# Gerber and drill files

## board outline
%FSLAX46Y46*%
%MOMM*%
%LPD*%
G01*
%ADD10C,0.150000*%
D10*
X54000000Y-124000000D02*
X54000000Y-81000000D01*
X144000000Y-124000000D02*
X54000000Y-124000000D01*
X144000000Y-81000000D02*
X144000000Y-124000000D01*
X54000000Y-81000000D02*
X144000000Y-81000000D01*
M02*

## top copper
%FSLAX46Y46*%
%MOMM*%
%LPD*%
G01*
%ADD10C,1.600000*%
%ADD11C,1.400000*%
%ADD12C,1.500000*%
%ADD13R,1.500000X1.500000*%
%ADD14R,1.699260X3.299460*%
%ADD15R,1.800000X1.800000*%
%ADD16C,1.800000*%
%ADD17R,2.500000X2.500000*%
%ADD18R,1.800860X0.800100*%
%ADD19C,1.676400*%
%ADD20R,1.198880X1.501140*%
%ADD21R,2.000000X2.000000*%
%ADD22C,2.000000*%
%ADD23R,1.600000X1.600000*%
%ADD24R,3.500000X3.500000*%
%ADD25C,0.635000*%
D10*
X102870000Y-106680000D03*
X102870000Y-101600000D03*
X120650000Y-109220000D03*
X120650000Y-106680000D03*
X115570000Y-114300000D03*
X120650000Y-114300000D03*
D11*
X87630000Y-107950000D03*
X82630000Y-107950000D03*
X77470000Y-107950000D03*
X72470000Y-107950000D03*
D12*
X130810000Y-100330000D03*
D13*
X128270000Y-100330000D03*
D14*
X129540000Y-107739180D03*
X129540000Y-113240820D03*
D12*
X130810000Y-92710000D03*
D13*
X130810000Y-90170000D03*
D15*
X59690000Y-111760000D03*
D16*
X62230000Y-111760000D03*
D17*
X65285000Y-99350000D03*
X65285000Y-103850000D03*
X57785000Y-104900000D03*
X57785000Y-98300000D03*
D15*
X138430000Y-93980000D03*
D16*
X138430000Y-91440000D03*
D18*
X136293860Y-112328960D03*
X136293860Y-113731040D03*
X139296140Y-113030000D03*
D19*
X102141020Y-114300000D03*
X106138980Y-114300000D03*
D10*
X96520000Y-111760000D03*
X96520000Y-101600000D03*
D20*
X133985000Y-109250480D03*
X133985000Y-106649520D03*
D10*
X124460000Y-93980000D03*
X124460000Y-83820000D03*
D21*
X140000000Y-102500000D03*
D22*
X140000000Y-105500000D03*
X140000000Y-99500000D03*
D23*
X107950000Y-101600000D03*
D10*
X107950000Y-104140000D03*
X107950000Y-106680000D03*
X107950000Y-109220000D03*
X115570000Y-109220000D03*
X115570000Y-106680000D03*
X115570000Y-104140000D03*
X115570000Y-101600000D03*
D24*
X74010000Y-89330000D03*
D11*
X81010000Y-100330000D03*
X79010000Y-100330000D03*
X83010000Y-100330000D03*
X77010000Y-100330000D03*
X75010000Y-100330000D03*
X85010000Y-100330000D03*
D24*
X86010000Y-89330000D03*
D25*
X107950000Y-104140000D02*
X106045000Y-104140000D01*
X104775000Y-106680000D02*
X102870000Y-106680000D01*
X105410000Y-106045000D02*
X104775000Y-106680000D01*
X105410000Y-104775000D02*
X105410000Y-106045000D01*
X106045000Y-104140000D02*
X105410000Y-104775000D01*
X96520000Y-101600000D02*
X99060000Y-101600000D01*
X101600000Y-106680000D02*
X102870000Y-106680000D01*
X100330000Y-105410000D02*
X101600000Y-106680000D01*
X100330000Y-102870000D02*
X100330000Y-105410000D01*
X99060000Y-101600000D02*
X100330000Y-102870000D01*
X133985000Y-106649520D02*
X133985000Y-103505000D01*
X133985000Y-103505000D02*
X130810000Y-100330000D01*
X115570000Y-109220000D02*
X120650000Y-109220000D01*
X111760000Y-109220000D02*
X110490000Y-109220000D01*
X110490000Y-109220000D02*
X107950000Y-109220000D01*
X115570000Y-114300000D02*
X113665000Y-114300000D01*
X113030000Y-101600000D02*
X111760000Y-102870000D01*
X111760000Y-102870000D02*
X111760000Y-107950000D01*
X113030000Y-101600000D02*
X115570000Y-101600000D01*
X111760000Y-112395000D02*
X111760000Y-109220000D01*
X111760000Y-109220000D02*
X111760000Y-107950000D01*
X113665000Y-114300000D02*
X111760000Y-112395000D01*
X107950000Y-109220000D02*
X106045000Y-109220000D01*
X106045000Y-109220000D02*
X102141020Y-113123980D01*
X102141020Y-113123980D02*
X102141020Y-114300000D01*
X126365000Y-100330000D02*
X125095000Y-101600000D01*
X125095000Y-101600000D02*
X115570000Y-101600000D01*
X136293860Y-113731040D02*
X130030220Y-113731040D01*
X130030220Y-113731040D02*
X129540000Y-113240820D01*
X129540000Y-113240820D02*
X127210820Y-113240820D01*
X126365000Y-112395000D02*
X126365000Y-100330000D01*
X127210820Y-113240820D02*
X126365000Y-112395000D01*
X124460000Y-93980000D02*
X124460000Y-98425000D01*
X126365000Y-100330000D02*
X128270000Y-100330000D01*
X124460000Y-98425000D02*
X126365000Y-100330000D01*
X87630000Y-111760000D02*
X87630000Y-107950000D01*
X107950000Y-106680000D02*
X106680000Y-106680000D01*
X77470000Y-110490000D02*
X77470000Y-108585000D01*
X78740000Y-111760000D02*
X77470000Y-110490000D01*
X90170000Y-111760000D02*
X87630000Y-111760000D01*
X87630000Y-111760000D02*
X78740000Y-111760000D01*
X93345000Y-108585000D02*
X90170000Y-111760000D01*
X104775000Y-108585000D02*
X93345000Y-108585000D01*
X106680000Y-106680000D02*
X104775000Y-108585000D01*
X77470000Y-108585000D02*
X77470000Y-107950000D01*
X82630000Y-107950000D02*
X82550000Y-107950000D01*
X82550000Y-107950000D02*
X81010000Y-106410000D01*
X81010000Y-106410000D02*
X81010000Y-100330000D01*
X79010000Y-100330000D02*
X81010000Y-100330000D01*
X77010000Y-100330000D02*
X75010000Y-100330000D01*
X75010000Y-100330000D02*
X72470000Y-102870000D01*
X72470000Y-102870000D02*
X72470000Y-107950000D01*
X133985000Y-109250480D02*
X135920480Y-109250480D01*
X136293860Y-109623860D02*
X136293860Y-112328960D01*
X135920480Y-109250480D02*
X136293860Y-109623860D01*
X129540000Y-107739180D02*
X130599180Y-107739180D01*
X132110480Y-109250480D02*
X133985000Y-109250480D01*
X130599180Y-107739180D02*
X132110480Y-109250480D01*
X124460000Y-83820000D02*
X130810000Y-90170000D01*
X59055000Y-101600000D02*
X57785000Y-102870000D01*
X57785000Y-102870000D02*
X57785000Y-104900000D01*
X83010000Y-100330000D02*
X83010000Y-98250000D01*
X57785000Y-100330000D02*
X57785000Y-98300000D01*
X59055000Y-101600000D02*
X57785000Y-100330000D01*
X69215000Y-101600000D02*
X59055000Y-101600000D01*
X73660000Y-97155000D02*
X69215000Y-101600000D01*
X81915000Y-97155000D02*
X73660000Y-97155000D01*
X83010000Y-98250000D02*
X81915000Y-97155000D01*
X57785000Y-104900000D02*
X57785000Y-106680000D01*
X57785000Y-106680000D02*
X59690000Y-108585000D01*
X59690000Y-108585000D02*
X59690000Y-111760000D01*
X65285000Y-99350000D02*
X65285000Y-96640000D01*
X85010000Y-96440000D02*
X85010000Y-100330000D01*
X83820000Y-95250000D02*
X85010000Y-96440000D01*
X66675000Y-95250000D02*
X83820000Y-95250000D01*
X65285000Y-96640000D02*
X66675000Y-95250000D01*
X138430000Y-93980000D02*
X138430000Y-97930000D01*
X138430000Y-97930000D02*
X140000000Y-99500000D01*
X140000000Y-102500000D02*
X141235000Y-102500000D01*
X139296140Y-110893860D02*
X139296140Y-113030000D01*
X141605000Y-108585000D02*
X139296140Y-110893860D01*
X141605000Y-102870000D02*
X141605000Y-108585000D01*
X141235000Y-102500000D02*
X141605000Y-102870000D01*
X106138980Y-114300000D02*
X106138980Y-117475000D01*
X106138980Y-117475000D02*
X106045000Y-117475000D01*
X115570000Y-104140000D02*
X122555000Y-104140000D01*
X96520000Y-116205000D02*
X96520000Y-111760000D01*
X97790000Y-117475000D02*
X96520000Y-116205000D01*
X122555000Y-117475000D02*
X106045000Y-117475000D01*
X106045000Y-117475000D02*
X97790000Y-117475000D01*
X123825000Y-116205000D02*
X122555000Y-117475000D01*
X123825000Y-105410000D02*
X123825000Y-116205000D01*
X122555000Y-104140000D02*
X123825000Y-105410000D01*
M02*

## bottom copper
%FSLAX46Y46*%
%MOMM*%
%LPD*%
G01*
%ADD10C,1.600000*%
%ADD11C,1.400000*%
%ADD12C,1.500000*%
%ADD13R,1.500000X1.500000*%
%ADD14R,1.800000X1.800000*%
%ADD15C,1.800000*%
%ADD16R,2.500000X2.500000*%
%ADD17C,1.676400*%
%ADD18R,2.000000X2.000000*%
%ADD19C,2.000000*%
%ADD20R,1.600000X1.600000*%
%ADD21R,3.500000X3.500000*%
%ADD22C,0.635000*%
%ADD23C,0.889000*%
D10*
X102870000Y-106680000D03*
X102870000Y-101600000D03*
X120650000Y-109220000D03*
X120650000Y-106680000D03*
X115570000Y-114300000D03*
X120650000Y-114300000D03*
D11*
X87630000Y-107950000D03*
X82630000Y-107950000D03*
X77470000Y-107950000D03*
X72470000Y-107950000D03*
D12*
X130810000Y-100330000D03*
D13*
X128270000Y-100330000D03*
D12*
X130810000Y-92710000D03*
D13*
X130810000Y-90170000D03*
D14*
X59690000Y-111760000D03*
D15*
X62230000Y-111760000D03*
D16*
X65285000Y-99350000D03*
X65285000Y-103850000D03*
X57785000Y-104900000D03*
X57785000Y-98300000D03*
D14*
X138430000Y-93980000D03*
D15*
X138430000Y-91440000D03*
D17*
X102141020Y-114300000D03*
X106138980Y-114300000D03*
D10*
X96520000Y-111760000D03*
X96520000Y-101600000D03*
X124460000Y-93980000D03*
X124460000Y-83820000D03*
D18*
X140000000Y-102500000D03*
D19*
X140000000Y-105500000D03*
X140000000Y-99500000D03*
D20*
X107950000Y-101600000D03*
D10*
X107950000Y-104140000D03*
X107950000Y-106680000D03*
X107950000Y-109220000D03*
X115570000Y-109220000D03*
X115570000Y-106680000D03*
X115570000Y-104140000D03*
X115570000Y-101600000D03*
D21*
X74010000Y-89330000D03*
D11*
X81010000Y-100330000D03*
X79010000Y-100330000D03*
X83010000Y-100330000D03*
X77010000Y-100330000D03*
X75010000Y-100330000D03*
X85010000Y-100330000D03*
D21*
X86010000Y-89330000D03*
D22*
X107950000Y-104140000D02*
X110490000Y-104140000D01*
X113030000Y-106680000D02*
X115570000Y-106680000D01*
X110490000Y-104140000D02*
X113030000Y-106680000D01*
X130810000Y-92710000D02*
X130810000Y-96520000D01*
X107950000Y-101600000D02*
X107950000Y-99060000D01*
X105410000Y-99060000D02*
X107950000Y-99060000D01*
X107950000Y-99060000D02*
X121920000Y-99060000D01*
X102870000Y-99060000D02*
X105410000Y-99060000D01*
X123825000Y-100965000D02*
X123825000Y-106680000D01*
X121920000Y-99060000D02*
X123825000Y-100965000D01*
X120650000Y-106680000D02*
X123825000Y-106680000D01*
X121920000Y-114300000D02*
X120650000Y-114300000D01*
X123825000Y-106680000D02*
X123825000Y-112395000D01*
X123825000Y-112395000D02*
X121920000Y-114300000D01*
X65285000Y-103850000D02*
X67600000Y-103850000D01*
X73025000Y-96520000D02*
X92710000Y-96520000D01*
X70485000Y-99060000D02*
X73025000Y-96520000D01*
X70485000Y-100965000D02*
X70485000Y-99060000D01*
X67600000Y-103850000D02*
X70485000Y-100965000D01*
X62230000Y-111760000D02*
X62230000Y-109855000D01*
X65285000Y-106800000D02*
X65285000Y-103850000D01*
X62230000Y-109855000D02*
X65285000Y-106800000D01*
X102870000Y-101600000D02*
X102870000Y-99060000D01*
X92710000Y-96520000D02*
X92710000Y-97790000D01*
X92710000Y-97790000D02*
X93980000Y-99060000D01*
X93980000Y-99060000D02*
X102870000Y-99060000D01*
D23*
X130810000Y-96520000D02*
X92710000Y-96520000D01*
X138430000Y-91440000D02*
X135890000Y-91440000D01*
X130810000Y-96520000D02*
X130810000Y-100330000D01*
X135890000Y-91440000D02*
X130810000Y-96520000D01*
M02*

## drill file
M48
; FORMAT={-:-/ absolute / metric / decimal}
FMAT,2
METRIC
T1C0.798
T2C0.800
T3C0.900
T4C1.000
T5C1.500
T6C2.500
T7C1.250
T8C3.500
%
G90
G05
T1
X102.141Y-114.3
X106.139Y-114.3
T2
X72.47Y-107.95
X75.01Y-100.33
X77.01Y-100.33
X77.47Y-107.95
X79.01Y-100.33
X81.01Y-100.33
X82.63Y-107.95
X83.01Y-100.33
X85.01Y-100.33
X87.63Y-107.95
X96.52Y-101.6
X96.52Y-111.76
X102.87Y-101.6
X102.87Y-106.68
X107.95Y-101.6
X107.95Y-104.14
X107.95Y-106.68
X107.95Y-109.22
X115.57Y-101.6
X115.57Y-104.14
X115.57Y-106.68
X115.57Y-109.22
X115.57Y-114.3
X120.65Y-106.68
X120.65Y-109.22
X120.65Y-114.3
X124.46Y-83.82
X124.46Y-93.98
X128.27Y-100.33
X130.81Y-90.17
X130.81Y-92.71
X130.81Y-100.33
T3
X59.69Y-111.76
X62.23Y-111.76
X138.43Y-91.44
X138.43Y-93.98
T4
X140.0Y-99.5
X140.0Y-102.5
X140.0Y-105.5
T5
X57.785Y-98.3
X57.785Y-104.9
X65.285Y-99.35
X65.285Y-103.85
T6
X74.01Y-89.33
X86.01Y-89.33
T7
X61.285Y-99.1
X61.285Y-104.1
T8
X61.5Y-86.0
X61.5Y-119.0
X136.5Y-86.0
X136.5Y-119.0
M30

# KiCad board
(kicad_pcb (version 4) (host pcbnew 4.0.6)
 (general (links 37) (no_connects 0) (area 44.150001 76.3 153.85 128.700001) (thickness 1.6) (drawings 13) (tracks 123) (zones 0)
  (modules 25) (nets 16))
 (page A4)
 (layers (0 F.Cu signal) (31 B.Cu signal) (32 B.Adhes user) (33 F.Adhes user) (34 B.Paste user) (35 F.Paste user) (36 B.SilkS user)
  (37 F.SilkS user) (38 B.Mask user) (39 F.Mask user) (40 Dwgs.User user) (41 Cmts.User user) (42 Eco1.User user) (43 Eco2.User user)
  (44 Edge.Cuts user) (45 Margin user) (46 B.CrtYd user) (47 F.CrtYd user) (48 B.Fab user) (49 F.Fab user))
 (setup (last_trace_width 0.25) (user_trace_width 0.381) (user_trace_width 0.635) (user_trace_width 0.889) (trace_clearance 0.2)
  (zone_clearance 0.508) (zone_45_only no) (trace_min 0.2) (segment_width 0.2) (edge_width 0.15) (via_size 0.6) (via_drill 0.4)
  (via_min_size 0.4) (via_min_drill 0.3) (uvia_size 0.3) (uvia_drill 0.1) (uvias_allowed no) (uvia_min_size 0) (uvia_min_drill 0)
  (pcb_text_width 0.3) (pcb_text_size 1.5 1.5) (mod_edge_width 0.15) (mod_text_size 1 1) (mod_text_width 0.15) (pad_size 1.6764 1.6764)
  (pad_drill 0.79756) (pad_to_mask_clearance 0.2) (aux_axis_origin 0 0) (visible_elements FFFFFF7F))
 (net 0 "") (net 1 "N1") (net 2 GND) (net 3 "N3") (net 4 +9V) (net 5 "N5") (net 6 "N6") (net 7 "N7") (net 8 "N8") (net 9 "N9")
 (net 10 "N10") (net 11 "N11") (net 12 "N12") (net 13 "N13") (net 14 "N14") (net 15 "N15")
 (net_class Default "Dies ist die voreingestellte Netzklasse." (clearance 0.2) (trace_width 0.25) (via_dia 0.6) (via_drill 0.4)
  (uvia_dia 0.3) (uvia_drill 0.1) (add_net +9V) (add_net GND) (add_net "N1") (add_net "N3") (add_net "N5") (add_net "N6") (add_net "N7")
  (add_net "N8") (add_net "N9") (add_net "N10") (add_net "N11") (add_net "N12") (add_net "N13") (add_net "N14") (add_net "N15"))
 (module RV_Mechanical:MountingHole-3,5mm (layer F.Cu) (at 136.5 86)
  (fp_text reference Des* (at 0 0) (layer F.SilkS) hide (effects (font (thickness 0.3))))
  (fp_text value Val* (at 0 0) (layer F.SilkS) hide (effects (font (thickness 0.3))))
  (pad "" np_thru_hole circle (at 0 0) (size 3.5 3.5) (drill 3.5) (layers *.Cu *.Mask F.SilkS)))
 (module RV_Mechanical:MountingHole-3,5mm (layer F.Cu) (at 61.5 119)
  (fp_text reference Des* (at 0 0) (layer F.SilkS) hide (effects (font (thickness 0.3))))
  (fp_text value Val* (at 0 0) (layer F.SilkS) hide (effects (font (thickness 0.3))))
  (pad "" np_thru_hole circle (at 0 0) (size 3.5 3.5) (drill 3.5) (layers *.Cu *.Mask F.SilkS)))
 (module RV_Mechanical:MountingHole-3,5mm (layer F.Cu) (at 136.5 119)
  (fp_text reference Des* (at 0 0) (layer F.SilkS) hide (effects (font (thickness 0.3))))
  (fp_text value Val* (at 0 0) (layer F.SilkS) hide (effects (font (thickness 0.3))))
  (pad "" np_thru_hole circle (at 0 0) (size 3.5 3.5) (drill 3.5) (layers *.Cu *.Mask F.SilkS)))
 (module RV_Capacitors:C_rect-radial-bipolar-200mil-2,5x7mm (layer F.Cu) (at 102.87 104.14 90)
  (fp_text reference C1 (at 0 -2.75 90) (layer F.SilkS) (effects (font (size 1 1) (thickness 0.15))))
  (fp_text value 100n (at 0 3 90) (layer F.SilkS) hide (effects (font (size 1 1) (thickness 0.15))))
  (pad 1 thru_hole circle (at -2.54 0 90) (size 1.6 1.6) (drill 0.8) (layers *.Cu *.Mask F.SilkS) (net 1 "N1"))
  (pad 2 thru_hole circle (at 2.54 0 90) (size 1.6 1.6) (drill 0.8) (layers *.Cu *.Mask F.SilkS) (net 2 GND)))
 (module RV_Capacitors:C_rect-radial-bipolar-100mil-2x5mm (layer F.Cu) (at 120.65 107.95 90)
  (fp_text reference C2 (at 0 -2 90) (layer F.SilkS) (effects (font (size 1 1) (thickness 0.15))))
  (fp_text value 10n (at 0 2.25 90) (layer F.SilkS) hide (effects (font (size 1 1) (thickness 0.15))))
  (pad 1 thru_hole circle (at -1.27 0 90) (size 1.6 1.6) (drill 0.8) (layers *.Cu *.Mask F.SilkS) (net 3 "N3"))
  (pad 2 thru_hole circle (at 1.27 0 90) (size 1.6 1.6) (drill 0.8) (layers *.Cu *.Mask F.SilkS) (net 2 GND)))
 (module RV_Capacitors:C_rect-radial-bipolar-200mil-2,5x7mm (layer F.Cu) (at 118.11 114.3)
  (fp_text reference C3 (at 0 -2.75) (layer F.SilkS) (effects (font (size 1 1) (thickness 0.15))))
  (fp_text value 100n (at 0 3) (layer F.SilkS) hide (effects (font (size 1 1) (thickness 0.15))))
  (pad 1 thru_hole circle (at -2.54 0) (size 1.6 1.6) (drill 0.8) (layers *.Cu *.Mask F.SilkS) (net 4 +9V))
  (pad 2 thru_hole circle (at 2.54 0) (size 1.6 1.6) (drill 0.8) (layers *.Cu *.Mask F.SilkS) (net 2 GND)))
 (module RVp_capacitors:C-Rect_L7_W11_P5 (layer F.Cu) (at 87.63 107.95 180)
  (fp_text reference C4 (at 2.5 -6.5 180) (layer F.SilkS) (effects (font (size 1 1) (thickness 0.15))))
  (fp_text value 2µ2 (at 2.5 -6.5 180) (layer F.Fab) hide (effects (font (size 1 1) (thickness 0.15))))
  (pad 1 thru_hole circle (at 0 0 180) (size 1.4 1.4) (drill 0.8) (layers *.Cu *.Mask) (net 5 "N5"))
  (pad 2 thru_hole circle (at 5 0 180) (size 1.4 1.4) (drill 0.8) (layers *.Cu *.Mask) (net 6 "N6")))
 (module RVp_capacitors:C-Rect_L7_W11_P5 (layer F.Cu) (at 77.47 107.95 180)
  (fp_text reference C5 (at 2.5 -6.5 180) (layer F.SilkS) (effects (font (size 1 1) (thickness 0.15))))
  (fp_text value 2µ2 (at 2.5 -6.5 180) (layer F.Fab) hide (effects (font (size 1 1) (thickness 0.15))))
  (pad 1 thru_hole circle (at 0 0 180) (size 1.4 1.4) (drill 0.8) (layers *.Cu *.Mask) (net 5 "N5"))
  (pad 2 thru_hole circle (at 5 0 180) (size 1.4 1.4) (drill 0.8) (layers *.Cu *.Mask) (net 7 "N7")))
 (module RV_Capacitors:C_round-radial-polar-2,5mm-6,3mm (layer F.Cu) (at 129.54 100.33)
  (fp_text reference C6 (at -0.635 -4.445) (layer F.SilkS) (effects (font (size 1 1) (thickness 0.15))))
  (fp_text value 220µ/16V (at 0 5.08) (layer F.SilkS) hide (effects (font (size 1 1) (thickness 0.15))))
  (pad 2 thru_hole circle (at 1.27 0) (size 1.5 1.5) (drill 0.8) (layers *.Cu *.Mask F.SilkS) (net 2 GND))
  (pad 1 thru_hole rect (at -1.27 0) (size 1.5 1.5) (drill 0.8) (layers *.Cu *.Mask F.SilkS) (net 4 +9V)))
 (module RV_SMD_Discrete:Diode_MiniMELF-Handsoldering (layer F.Cu) (at 129.54 110.49 270)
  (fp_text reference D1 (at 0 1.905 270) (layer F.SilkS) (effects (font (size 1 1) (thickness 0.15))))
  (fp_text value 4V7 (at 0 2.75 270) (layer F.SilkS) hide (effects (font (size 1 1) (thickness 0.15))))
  (pad 1 smd rect (at -2.75082 0 270) (size 3.29946 1.69926) (layers F.Cu F.Paste F.Mask) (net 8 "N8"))
  (pad 2 smd rect (at 2.75082 0 270) (size 3.29946 1.69926) (layers F.Cu F.Paste F.Mask) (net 4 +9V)))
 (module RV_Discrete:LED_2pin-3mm (layer F.Cu) (at 130.81 91.44 270)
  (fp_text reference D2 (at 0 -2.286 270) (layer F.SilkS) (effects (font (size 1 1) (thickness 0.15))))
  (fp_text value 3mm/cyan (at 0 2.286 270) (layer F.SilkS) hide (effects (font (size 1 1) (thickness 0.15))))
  (pad 2 thru_hole circle (at 1.27 0 270) (size 1.5 1.5) (drill 0.8) (layers *.Cu *.Mask F.SilkS) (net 2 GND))
  (pad 1 thru_hole rect (at -1.27 0 270) (size 1.5 1.5) (drill 0.8) (layers *.Cu *.Mask F.SilkS) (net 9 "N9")))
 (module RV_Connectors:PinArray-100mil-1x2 (layer F.Cu) (at 60.96 111.76)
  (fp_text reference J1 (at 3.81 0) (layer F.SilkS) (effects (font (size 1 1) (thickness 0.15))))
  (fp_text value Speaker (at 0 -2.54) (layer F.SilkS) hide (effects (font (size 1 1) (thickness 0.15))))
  (pad 1 thru_hole rect (at -1.27 0) (size 1.8 1.8) (drill 0.9) (layers *.Cu *.Mask F.SilkS) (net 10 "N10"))
  (pad 2 thru_hole circle (at 1.27 0) (size 1.8 1.8) (drill 0.9) (layers *.Cu *.Mask F.SilkS) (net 2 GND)))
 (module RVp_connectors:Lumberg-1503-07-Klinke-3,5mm (layer F.Cu) (at 57.785 101.6 90)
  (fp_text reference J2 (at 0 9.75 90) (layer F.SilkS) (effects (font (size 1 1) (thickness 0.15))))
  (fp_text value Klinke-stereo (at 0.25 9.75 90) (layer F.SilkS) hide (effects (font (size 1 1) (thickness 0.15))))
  (pad 2 thru_hole rect (at 2.25 7.5 90) (size 2.5 2.5) (drill 1.5) (layers *.Cu *.Mask) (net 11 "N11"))
  (pad 1 thru_hole rect (at -2.25 7.5 90) (size 2.5 2.5) (drill 1.5) (layers *.Cu *.Mask) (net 2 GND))
  (pad "" np_thru_hole circle (at 2.5 3.5 90) (size 1.25 1.25) (drill 1.25) (layers *.Cu *.Mask))
  (pad "" np_thru_hole circle (at -2.5 3.5 90) (size 1.25 1.25) (drill 1.25) (layers *.Cu *.Mask))
  (pad 3 thru_hole rect (at -3.3 0 90) (size 2.5 2.5) (drill 1.5) (layers *.Cu *.Mask) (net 10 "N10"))
  (pad 3 thru_hole rect (at 3.3 0 90) (size 2.5 2.5) (drill 1.5) (layers *.Cu *.Mask) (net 10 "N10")))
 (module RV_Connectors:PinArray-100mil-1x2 (layer F.Cu) (at 138.43 92.71 90)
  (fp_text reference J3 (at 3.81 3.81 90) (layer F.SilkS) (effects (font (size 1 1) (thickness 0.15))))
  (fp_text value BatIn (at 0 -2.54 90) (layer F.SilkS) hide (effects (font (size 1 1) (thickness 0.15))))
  (pad 1 thru_hole rect (at -1.27 0 90) (size 1.8 1.8) (drill 0.9) (layers *.Cu *.Mask F.SilkS) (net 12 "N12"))
  (pad 2 thru_hole circle (at 1.27 0 90) (size 1.8 1.8) (drill 0.9) (layers *.Cu *.Mask F.SilkS) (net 2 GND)))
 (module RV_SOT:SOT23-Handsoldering (layer F.Cu) (at 137.795 113.03 270)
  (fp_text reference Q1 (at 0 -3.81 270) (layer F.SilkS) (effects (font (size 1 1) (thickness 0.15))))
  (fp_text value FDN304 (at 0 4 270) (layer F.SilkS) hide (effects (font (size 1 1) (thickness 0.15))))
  (pad 1 smd rect (at -0.70104 1.50114 270) (size 0.8001 1.80086) (layers F.Cu F.Paste F.Mask) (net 8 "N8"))
  (pad 2 smd rect (at 0.70104 1.50114 270) (size 0.8001 1.80086) (layers F.Cu F.Paste F.Mask) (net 4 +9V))
  (pad 3 smd rect (at 0 -1.50114 270) (size 0.8001 1.80086) (layers F.Cu F.Paste F.Mask) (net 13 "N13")))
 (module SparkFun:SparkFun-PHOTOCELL (layer F.Cu) (at 104.14 114.3)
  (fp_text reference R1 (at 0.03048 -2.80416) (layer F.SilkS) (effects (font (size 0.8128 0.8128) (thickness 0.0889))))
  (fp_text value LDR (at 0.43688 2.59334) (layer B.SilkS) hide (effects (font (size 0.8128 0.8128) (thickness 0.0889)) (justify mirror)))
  (pad 1 thru_hole circle (at -1.99898 0) (size 1.6764 1.6764) (drill 0.79756) (layers *.Cu *.Mask) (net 4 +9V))
  (pad 2 thru_hole circle (at 1.99898 0) (size 1.6764 1.6764) (drill 0.79756) (layers *.Cu *.Mask) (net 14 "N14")))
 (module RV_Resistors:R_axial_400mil (layer F.Cu) (at 96.52 106.68 90)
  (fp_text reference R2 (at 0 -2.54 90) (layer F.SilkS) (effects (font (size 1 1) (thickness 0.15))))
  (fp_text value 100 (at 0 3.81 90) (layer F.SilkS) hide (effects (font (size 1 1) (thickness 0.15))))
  (pad 1 thru_hole circle (at -5.08 0 90) (size 1.6 1.6) (drill 0.8) (layers *.Cu *.Mask) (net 14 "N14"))
  (pad 2 thru_hole circle (at 5.08 0 90) (size 1.6 1.6) (drill 0.8) (layers *.Cu *.Mask) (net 1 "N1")))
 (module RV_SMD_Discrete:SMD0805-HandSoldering (layer F.Cu) (at 133.985 107.95 90)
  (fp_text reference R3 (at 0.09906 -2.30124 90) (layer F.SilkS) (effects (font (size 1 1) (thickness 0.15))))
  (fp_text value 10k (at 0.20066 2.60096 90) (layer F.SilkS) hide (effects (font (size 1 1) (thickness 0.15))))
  (pad 1 smd rect (at -1.30048 0 90) (size 1.50114 1.19888) (layers F.Cu F.Paste F.Mask) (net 8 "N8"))
  (pad 2 smd rect (at 1.30048 0 90) (size 1.50114 1.19888) (layers F.Cu F.Paste F.Mask) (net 2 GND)))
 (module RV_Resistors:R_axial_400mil (layer F.Cu) (at 124.46 88.9 90)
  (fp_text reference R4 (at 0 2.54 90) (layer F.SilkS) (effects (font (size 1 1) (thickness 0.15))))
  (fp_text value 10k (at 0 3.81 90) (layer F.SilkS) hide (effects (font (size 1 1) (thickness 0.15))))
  (pad 1 thru_hole circle (at -5.08 0 90) (size 1.6 1.6) (drill 0.8) (layers *.Cu *.Mask) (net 4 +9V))
  (pad 2 thru_hole circle (at 5.08 0 90) (size 1.6 1.6) (drill 0.8) (layers *.Cu *.Mask) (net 9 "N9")))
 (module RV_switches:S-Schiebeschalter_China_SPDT (layer F.Cu) (at 140 102.5 90)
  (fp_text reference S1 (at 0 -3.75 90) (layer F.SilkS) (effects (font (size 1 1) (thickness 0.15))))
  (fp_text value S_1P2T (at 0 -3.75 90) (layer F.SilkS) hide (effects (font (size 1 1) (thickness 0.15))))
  (pad 2 thru_hole rect (at 0 0 90) (size 2 2) (drill 1) (layers *.Cu *.Mask) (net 13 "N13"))
  (pad 1 thru_hole circle (at -3 0 90) (size 2 2) (drill 1) (layers *.Cu *.Mask) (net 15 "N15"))
  (pad 3 thru_hole circle (at 3 0 90) (size 2 2) (drill 1) (layers *.Cu *.Mask) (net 12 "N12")))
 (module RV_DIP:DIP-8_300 (layer F.Cu) (at 111.76 105.41 270)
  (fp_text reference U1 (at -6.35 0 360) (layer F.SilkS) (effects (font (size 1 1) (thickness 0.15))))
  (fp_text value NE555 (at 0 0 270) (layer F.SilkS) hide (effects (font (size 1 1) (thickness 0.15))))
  (pad 1 thru_hole rect (at -3.81 3.81 270) (size 1.6 1.6) (drill 0.8) (layers *.Cu *.Mask F.SilkS) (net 2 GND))
  (pad 2 thru_hole circle (at -1.27 3.81 270) (size 1.6 1.6) (drill 0.8) (layers *.Cu *.Mask F.SilkS) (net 1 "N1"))
  (pad 3 thru_hole circle (at 1.27 3.81 270) (size 1.6 1.6) (drill 0.8) (layers *.Cu *.Mask F.SilkS) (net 5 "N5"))
  (pad 4 thru_hole circle (at 3.81 3.81 270) (size 1.6 1.6) (drill 0.8) (layers *.Cu *.Mask F.SilkS) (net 4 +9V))
  (pad 5 thru_hole circle (at 3.81 -3.81 270) (size 1.6 1.6) (drill 0.8) (layers *.Cu *.Mask F.SilkS) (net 3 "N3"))
  (pad 6 thru_hole circle (at 1.27 -3.81 270) (size 1.6 1.6) (drill 0.8) (layers *.Cu *.Mask F.SilkS) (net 1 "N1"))
  (pad 7 thru_hole circle (at -1.27 -3.81 270) (size 1.6 1.6) (drill 0.8) (layers *.Cu *.Mask F.SilkS) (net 14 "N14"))
  (pad 8 thru_hole circle (at -3.81 -3.81 270) (size 1.6 1.6) (drill 0.8) (layers *.Cu *.Mask F.SilkS) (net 4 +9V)))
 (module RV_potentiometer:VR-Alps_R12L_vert (layer F.Cu) (at 80.01 100.33)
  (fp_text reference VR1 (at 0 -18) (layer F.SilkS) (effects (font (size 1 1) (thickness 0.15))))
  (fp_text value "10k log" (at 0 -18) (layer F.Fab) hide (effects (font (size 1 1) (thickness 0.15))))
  (pad M thru_hole rect (at -6 -11) (size 3.5 3.5) (drill 2.5) (layers *.Cu *.Mask))
  (pad 2 thru_hole circle (at 1 0) (size 1.4 1.4) (drill 0.8) (layers *.Cu *.Mask) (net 6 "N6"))
  (pad 1 thru_hole circle (at -1 0) (size 1.4 1.4) (drill 0.8) (layers *.Cu *.Mask) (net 6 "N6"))
  (pad 3 thru_hole circle (at 3 0) (size 1.4 1.4) (drill 0.8) (layers *.Cu *.Mask) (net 10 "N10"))
  (pad 4 thru_hole circle (at -3 0) (size 1.4 1.4) (drill 0.8) (layers *.Cu *.Mask) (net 7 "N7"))
  (pad 5 thru_hole circle (at -5 0) (size 1.4 1.4) (drill 0.8) (layers *.Cu *.Mask) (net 7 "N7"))
  (pad 6 thru_hole circle (at 5 0) (size 1.4 1.4) (drill 0.8) (layers *.Cu *.Mask) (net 11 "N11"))
  (pad M thru_hole rect (at 6 -11) (size 3.5 3.5) (drill 2.5) (layers *.Cu *.Mask)))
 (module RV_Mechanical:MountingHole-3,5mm (layer F.Cu) (at 61.5 86)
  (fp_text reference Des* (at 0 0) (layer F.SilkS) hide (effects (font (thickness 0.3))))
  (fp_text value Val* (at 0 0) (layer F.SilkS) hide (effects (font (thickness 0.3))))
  (pad "" np_thru_hole circle (at 0 0) (size 3.5 3.5) (drill 3.5) (layers *.Cu *.Mask F.SilkS)))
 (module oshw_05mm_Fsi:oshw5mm (layer F.Cu) (at 85.09 118.745)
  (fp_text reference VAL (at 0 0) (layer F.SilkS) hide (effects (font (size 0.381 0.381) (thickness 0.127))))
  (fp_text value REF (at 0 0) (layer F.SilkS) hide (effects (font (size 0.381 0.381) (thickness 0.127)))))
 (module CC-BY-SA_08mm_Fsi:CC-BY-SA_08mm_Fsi (layer F.Cu) (at 74.93 118.745)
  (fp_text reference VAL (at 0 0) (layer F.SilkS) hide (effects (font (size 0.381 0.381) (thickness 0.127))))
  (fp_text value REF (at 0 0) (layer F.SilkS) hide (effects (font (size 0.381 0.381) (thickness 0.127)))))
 (gr_line (start 54 124) (end 54 81) (angle 90) (layer Edge.Cuts) (width 0.15))
 (gr_line (start 144 124) (end 54 124) (angle 90) (layer Edge.Cuts) (width 0.15))
 (gr_line (start 144 81) (end 144 124) (angle 90) (layer Edge.Cuts) (width 0.15))
 (gr_line (start 54 81) (end 144 81) (angle 90) (layer Edge.Cuts) (width 0.15))
 (segment (start 107.95 104.14) (end 110.49 104.14) (width 0.635) (layer B.Cu) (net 1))
 (segment (start 113.03 106.68) (end 115.57 106.68) (width 0.635) (layer B.Cu) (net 1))
 (segment (start 110.49 104.14) (end 113.03 106.68) (width 0.635) (layer B.Cu) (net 1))
 (segment (start 107.95 104.14) (end 106.045 104.14) (width 0.635) (layer F.Cu) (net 1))
 (segment (start 104.775 106.68) (end 102.87 106.68) (width 0.635) (layer F.Cu) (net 1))
 (segment (start 105.41 106.045) (end 104.775 106.68) (width 0.635) (layer F.Cu) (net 1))
 (segment (start 105.41 104.775) (end 105.41 106.045) (width 0.635) (layer F.Cu) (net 1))
 (segment (start 106.045 104.14) (end 105.41 104.775) (width 0.635) (layer F.Cu) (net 1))
 (segment (start 96.52 101.6) (end 99.06 101.6) (width 0.635) (layer F.Cu) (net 1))
 (segment (start 101.6 106.68) (end 102.87 106.68) (width 0.635) (layer F.Cu) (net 1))
 (segment (start 100.33 105.41) (end 101.6 106.68) (width 0.635) (layer F.Cu) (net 1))
 (segment (start 100.33 102.87) (end 100.33 105.41) (width 0.635) (layer F.Cu) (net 1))
 (segment (start 99.06 101.6) (end 100.33 102.87) (width 0.635) (layer F.Cu) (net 1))
 (segment (start 133.985 106.64952) (end 133.985 103.505) (width 0.635) (layer F.Cu) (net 2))
 (segment (start 133.985 103.505) (end 130.81 100.33) (width 0.635) (layer F.Cu) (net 2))
 (segment (start 130.81 92.71) (end 130.81 96.52) (width 0.635) (layer B.Cu) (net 2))
 (segment (start 107.95 101.6) (end 107.95 99.06) (width 0.635) (layer B.Cu) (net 2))
 (segment (start 105.41 99.06) (end 107.95 99.06) (width 0.635) (layer B.Cu) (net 2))
 (segment (start 107.95 99.06) (end 121.92 99.06) (width 0.635) (layer B.Cu) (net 2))
 (segment (start 102.87 99.06) (end 105.41 99.06) (width 0.635) (layer B.Cu) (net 2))
 (segment (start 123.825 100.965) (end 123.825 106.68) (width 0.635) (layer B.Cu) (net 2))
 (segment (start 121.92 99.06) (end 123.825 100.965) (width 0.635) (layer B.Cu) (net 2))
 (segment (start 120.65 106.68) (end 123.825 106.68) (width 0.635) (layer B.Cu) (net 2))
 (segment (start 121.92 114.3) (end 120.65 114.3) (width 0.635) (layer B.Cu) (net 2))
 (segment (start 123.825 106.68) (end 123.825 112.395) (width 0.635) (layer B.Cu) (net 2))
 (segment (start 123.825 112.395) (end 121.92 114.3) (width 0.635) (layer B.Cu) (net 2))
 (segment (start 65.285 103.85) (end 67.6 103.85) (width 0.635) (layer B.Cu) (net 2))
 (segment (start 73.025 96.52) (end 92.71 96.52) (width 0.635) (layer B.Cu) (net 2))
 (segment (start 70.485 99.06) (end 73.025 96.52) (width 0.635) (layer B.Cu) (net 2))
 (segment (start 70.485 100.965) (end 70.485 99.06) (width 0.635) (layer B.Cu) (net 2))
 (segment (start 67.6 103.85) (end 70.485 100.965) (width 0.635) (layer B.Cu) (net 2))
 (segment (start 62.23 111.76) (end 62.23 109.855) (width 0.635) (layer B.Cu) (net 2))
 (segment (start 65.285 106.8) (end 65.285 103.85) (width 0.635) (layer B.Cu) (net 2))
 (segment (start 62.23 109.855) (end 65.285 106.8) (width 0.635) (layer B.Cu) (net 2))
 (segment (start 102.87 101.6) (end 102.87 99.06) (width 0.635) (layer B.Cu) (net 2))
 (segment (start 92.71 96.52) (end 92.71 97.79) (width 0.635) (layer B.Cu) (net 2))
 (segment (start 92.71 97.79) (end 93.98 99.06) (width 0.635) (layer B.Cu) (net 2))
 (segment (start 93.98 99.06) (end 102.87 99.06) (width 0.635) (layer B.Cu) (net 2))
 (segment (start 130.81 96.52) (end 92.71 96.52) (width 0.889) (layer B.Cu) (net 2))
 (segment (start 138.43 91.44) (end 135.89 91.44) (width 0.889) (layer B.Cu) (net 2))
 (segment (start 130.81 96.52) (end 130.81 100.33) (width 0.889) (layer B.Cu) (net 2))
 (segment (start 135.89 91.44) (end 130.81 96.52) (width 0.889) (layer B.Cu) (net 2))
 (segment (start 115.57 109.22) (end 120.65 109.22) (width 0.635) (layer F.Cu) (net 3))
 (segment (start 111.76 109.22) (end 110.49 109.22) (width 0.635) (layer F.Cu) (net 4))
 (segment (start 110.49 109.22) (end 107.95 109.22) (width 0.635) (layer F.Cu) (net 4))
 (segment (start 115.57 114.3) (end 113.665 114.3) (width 0.635) (layer F.Cu) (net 4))
 (segment (start 113.03 101.6) (end 111.76 102.87) (width 0.635) (layer F.Cu) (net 4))
 (segment (start 111.76 102.87) (end 111.76 107.95) (width 0.635) (layer F.Cu) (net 4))
 (segment (start 113.03 101.6) (end 115.57 101.6) (width 0.635) (layer F.Cu) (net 4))
 (segment (start 111.76 112.395) (end 111.76 109.22) (width 0.635) (layer F.Cu) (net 4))
 (segment (start 111.76 109.22) (end 111.76 107.95) (width 0.635) (layer F.Cu) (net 4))
 (segment (start 113.665 114.3) (end 111.76 112.395) (width 0.635) (layer F.Cu) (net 4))
 (segment (start 107.95 109.22) (end 106.045 109.22) (width 0.635) (layer F.Cu) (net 4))
 (segment (start 106.045 109.22) (end 102.14102 113.12398) (width 0.635) (layer F.Cu) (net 4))
 (segment (start 102.14102 113.12398) (end 102.14102 114.3) (width 0.635) (layer F.Cu) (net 4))
 (segment (start 126.365 100.33) (end 125.095 101.6) (width 0.635) (layer F.Cu) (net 4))
 (segment (start 125.095 101.6) (end 115.57 101.6) (width 0.635) (layer F.Cu) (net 4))
 (segment (start 136.29386 113.73104) (end 130.03022 113.73104) (width 0.635) (layer F.Cu) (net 4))
 (segment (start 130.03022 113.73104) (end 129.54 113.24082) (width 0.635) (layer F.Cu) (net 4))
 (segment (start 129.54 113.24082) (end 127.21082 113.24082) (width 0.635) (layer F.Cu) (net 4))
 (segment (start 126.365 112.395) (end 126.365 100.33) (width 0.635) (layer F.Cu) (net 4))
 (segment (start 127.21082 113.24082) (end 126.365 112.395) (width 0.635) (layer F.Cu) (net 4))
 (segment (start 124.46 93.98) (end 124.46 98.425) (width 0.635) (layer F.Cu) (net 4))
 (segment (start 126.365 100.33) (end 128.27 100.33) (width 0.635) (layer F.Cu) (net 4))
 (segment (start 124.46 98.425) (end 126.365 100.33) (width 0.635) (layer F.Cu) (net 4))
 (segment (start 87.63 111.76) (end 87.63 107.95) (width 0.635) (layer F.Cu) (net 5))
 (segment (start 107.95 106.68) (end 106.68 106.68) (width 0.635) (layer F.Cu) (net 5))
 (segment (start 77.47 110.49) (end 77.47 108.585) (width 0.635) (layer F.Cu) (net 5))
 (segment (start 78.74 111.76) (end 77.47 110.49) (width 0.635) (layer F.Cu) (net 5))
 (segment (start 90.17 111.76) (end 87.63 111.76) (width 0.635) (layer F.Cu) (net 5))
 (segment (start 87.63 111.76) (end 78.74 111.76) (width 0.635) (layer F.Cu) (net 5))
 (segment (start 93.345 108.585) (end 90.17 111.76) (width 0.635) (layer F.Cu) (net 5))
 (segment (start 104.775 108.585) (end 93.345 108.585) (width 0.635) (layer F.Cu) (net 5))
 (segment (start 106.68 106.68) (end 104.775 108.585) (width 0.635) (layer F.Cu) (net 5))
 (segment (start 77.47 108.585) (end 77.47 107.95) (width 0.635) (layer F.Cu) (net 5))
 (segment (start 82.63 107.95) (end 82.55 107.95) (width 0.635) (layer F.Cu) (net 6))
 (segment (start 82.55 107.95) (end 81.01 106.41) (width 0.635) (layer F.Cu) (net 6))
 (segment (start 81.01 106.41) (end 81.01 100.33) (width 0.635) (layer F.Cu) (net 6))
 (segment (start 79.01 100.33) (end 81.01 100.33) (width 0.635) (layer F.Cu) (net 6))
 (segment (start 77.01 100.33) (end 75.01 100.33) (width 0.635) (layer F.Cu) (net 7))
 (segment (start 75.01 100.33) (end 72.47 102.87) (width 0.635) (layer F.Cu) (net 7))
 (segment (start 72.47 102.87) (end 72.47 107.95) (width 0.635) (layer F.Cu) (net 7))
 (segment (start 133.985 109.25048) (end 135.92048 109.25048) (width 0.635) (layer F.Cu) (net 8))
 (segment (start 136.29386 109.62386) (end 136.29386 112.32896) (width 0.635) (layer F.Cu) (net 8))
 (segment (start 135.92048 109.25048) (end 136.29386 109.62386) (width 0.635) (layer F.Cu) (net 8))
 (segment (start 129.54 107.73918) (end 130.59918 107.73918) (width 0.635) (layer F.Cu) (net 8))
 (segment (start 132.11048 109.25048) (end 133.985 109.25048) (width 0.635) (layer F.Cu) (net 8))
 (segment (start 130.59918 107.73918) (end 132.11048 109.25048) (width 0.635) (layer F.Cu) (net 8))
 (segment (start 124.46 83.82) (end 130.81 90.17) (width 0.635) (layer F.Cu) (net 9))
 (segment (start 59.055 101.6) (end 57.785 102.87) (width 0.635) (layer F.Cu) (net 10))
 (segment (start 57.785 102.87) (end 57.785 104.9) (width 0.635) (layer F.Cu) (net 10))
 (segment (start 83.01 100.33) (end 83.01 98.25) (width 0.635) (layer F.Cu) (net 10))
 (segment (start 57.785 100.33) (end 57.785 98.3) (width 0.635) (layer F.Cu) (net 10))
 (segment (start 59.055 101.6) (end 57.785 100.33) (width 0.635) (layer F.Cu) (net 10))
 (segment (start 69.215 101.6) (end 59.055 101.6) (width 0.635) (layer F.Cu) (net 10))
 (segment (start 73.66 97.155) (end 69.215 101.6) (width 0.635) (layer F.Cu) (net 10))
 (segment (start 81.915 97.155) (end 73.66 97.155) (width 0.635) (layer F.Cu) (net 10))
 (segment (start 83.01 98.25) (end 81.915 97.155) (width 0.635) (layer F.Cu) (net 10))
 (segment (start 57.785 104.9) (end 57.785 106.68) (width 0.635) (layer F.Cu) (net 10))
 (segment (start 57.785 106.68) (end 59.69 108.585) (width 0.635) (layer F.Cu) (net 10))
 (segment (start 59.69 108.585) (end 59.69 111.76) (width 0.635) (layer F.Cu) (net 10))
 (segment (start 65.285 99.35) (end 65.285 96.64) (width 0.635) (layer F.Cu) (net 11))
 (segment (start 85.01 96.44) (end 85.01 100.33) (width 0.635) (layer F.Cu) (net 11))
 (segment (start 83.82 95.25) (end 85.01 96.44) (width 0.635) (layer F.Cu) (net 11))
 (segment (start 66.675 95.25) (end 83.82 95.25) (width 0.635) (layer F.Cu) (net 11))
 (segment (start 65.285 96.64) (end 66.675 95.25) (width 0.635) (layer F.Cu) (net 11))
 (segment (start 138.43 93.98) (end 138.43 97.93) (width 0.635) (layer F.Cu) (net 12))
 (segment (start 138.43 97.93) (end 140 99.5) (width 0.635) (layer F.Cu) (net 12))
 (segment (start 140 102.5) (end 141.235 102.5) (width 0.635) (layer F.Cu) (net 13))
 (segment (start 139.29614 110.89386) (end 139.29614 113.03) (width 0.635) (layer F.Cu) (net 13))
 (segment (start 141.605 108.585) (end 139.29614 110.89386) (width 0.635) (layer F.Cu) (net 13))
 (segment (start 141.605 102.87) (end 141.605 108.585) (width 0.635) (layer F.Cu) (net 13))
 (segment (start 141.235 102.5) (end 141.605 102.87) (width 0.635) (layer F.Cu) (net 13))
 (segment (start 106.13898 114.3) (end 106.13898 117.475) (width 0.635) (layer F.Cu) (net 14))
 (segment (start 106.13898 117.475) (end 106.045 117.475) (width 0.635) (layer F.Cu) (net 14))
 (segment (start 115.57 104.14) (end 122.555 104.14) (width 0.635) (layer F.Cu) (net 14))
 (segment (start 96.52 116.205) (end 96.52 111.76) (width 0.635) (layer F.Cu) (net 14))
 (segment (start 97.79 117.475) (end 96.52 116.205) (width 0.635) (layer F.Cu) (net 14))
 (segment (start 122.555 117.475) (end 106.045 117.475) (width 0.635) (layer F.Cu) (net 14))
 (segment (start 106.045 117.475) (end 97.79 117.475) (width 0.635) (layer F.Cu) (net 14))
 (segment (start 123.825 116.205) (end 122.555 117.475) (width 0.635) (layer F.Cu) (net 14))
 (segment (start 123.825 105.41) (end 123.825 116.205) (width 0.635) (layer F.Cu) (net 14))
 (segment (start 122.555 104.14) (end 123.825 105.41) (width 0.635) (layer F.Cu) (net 14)))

